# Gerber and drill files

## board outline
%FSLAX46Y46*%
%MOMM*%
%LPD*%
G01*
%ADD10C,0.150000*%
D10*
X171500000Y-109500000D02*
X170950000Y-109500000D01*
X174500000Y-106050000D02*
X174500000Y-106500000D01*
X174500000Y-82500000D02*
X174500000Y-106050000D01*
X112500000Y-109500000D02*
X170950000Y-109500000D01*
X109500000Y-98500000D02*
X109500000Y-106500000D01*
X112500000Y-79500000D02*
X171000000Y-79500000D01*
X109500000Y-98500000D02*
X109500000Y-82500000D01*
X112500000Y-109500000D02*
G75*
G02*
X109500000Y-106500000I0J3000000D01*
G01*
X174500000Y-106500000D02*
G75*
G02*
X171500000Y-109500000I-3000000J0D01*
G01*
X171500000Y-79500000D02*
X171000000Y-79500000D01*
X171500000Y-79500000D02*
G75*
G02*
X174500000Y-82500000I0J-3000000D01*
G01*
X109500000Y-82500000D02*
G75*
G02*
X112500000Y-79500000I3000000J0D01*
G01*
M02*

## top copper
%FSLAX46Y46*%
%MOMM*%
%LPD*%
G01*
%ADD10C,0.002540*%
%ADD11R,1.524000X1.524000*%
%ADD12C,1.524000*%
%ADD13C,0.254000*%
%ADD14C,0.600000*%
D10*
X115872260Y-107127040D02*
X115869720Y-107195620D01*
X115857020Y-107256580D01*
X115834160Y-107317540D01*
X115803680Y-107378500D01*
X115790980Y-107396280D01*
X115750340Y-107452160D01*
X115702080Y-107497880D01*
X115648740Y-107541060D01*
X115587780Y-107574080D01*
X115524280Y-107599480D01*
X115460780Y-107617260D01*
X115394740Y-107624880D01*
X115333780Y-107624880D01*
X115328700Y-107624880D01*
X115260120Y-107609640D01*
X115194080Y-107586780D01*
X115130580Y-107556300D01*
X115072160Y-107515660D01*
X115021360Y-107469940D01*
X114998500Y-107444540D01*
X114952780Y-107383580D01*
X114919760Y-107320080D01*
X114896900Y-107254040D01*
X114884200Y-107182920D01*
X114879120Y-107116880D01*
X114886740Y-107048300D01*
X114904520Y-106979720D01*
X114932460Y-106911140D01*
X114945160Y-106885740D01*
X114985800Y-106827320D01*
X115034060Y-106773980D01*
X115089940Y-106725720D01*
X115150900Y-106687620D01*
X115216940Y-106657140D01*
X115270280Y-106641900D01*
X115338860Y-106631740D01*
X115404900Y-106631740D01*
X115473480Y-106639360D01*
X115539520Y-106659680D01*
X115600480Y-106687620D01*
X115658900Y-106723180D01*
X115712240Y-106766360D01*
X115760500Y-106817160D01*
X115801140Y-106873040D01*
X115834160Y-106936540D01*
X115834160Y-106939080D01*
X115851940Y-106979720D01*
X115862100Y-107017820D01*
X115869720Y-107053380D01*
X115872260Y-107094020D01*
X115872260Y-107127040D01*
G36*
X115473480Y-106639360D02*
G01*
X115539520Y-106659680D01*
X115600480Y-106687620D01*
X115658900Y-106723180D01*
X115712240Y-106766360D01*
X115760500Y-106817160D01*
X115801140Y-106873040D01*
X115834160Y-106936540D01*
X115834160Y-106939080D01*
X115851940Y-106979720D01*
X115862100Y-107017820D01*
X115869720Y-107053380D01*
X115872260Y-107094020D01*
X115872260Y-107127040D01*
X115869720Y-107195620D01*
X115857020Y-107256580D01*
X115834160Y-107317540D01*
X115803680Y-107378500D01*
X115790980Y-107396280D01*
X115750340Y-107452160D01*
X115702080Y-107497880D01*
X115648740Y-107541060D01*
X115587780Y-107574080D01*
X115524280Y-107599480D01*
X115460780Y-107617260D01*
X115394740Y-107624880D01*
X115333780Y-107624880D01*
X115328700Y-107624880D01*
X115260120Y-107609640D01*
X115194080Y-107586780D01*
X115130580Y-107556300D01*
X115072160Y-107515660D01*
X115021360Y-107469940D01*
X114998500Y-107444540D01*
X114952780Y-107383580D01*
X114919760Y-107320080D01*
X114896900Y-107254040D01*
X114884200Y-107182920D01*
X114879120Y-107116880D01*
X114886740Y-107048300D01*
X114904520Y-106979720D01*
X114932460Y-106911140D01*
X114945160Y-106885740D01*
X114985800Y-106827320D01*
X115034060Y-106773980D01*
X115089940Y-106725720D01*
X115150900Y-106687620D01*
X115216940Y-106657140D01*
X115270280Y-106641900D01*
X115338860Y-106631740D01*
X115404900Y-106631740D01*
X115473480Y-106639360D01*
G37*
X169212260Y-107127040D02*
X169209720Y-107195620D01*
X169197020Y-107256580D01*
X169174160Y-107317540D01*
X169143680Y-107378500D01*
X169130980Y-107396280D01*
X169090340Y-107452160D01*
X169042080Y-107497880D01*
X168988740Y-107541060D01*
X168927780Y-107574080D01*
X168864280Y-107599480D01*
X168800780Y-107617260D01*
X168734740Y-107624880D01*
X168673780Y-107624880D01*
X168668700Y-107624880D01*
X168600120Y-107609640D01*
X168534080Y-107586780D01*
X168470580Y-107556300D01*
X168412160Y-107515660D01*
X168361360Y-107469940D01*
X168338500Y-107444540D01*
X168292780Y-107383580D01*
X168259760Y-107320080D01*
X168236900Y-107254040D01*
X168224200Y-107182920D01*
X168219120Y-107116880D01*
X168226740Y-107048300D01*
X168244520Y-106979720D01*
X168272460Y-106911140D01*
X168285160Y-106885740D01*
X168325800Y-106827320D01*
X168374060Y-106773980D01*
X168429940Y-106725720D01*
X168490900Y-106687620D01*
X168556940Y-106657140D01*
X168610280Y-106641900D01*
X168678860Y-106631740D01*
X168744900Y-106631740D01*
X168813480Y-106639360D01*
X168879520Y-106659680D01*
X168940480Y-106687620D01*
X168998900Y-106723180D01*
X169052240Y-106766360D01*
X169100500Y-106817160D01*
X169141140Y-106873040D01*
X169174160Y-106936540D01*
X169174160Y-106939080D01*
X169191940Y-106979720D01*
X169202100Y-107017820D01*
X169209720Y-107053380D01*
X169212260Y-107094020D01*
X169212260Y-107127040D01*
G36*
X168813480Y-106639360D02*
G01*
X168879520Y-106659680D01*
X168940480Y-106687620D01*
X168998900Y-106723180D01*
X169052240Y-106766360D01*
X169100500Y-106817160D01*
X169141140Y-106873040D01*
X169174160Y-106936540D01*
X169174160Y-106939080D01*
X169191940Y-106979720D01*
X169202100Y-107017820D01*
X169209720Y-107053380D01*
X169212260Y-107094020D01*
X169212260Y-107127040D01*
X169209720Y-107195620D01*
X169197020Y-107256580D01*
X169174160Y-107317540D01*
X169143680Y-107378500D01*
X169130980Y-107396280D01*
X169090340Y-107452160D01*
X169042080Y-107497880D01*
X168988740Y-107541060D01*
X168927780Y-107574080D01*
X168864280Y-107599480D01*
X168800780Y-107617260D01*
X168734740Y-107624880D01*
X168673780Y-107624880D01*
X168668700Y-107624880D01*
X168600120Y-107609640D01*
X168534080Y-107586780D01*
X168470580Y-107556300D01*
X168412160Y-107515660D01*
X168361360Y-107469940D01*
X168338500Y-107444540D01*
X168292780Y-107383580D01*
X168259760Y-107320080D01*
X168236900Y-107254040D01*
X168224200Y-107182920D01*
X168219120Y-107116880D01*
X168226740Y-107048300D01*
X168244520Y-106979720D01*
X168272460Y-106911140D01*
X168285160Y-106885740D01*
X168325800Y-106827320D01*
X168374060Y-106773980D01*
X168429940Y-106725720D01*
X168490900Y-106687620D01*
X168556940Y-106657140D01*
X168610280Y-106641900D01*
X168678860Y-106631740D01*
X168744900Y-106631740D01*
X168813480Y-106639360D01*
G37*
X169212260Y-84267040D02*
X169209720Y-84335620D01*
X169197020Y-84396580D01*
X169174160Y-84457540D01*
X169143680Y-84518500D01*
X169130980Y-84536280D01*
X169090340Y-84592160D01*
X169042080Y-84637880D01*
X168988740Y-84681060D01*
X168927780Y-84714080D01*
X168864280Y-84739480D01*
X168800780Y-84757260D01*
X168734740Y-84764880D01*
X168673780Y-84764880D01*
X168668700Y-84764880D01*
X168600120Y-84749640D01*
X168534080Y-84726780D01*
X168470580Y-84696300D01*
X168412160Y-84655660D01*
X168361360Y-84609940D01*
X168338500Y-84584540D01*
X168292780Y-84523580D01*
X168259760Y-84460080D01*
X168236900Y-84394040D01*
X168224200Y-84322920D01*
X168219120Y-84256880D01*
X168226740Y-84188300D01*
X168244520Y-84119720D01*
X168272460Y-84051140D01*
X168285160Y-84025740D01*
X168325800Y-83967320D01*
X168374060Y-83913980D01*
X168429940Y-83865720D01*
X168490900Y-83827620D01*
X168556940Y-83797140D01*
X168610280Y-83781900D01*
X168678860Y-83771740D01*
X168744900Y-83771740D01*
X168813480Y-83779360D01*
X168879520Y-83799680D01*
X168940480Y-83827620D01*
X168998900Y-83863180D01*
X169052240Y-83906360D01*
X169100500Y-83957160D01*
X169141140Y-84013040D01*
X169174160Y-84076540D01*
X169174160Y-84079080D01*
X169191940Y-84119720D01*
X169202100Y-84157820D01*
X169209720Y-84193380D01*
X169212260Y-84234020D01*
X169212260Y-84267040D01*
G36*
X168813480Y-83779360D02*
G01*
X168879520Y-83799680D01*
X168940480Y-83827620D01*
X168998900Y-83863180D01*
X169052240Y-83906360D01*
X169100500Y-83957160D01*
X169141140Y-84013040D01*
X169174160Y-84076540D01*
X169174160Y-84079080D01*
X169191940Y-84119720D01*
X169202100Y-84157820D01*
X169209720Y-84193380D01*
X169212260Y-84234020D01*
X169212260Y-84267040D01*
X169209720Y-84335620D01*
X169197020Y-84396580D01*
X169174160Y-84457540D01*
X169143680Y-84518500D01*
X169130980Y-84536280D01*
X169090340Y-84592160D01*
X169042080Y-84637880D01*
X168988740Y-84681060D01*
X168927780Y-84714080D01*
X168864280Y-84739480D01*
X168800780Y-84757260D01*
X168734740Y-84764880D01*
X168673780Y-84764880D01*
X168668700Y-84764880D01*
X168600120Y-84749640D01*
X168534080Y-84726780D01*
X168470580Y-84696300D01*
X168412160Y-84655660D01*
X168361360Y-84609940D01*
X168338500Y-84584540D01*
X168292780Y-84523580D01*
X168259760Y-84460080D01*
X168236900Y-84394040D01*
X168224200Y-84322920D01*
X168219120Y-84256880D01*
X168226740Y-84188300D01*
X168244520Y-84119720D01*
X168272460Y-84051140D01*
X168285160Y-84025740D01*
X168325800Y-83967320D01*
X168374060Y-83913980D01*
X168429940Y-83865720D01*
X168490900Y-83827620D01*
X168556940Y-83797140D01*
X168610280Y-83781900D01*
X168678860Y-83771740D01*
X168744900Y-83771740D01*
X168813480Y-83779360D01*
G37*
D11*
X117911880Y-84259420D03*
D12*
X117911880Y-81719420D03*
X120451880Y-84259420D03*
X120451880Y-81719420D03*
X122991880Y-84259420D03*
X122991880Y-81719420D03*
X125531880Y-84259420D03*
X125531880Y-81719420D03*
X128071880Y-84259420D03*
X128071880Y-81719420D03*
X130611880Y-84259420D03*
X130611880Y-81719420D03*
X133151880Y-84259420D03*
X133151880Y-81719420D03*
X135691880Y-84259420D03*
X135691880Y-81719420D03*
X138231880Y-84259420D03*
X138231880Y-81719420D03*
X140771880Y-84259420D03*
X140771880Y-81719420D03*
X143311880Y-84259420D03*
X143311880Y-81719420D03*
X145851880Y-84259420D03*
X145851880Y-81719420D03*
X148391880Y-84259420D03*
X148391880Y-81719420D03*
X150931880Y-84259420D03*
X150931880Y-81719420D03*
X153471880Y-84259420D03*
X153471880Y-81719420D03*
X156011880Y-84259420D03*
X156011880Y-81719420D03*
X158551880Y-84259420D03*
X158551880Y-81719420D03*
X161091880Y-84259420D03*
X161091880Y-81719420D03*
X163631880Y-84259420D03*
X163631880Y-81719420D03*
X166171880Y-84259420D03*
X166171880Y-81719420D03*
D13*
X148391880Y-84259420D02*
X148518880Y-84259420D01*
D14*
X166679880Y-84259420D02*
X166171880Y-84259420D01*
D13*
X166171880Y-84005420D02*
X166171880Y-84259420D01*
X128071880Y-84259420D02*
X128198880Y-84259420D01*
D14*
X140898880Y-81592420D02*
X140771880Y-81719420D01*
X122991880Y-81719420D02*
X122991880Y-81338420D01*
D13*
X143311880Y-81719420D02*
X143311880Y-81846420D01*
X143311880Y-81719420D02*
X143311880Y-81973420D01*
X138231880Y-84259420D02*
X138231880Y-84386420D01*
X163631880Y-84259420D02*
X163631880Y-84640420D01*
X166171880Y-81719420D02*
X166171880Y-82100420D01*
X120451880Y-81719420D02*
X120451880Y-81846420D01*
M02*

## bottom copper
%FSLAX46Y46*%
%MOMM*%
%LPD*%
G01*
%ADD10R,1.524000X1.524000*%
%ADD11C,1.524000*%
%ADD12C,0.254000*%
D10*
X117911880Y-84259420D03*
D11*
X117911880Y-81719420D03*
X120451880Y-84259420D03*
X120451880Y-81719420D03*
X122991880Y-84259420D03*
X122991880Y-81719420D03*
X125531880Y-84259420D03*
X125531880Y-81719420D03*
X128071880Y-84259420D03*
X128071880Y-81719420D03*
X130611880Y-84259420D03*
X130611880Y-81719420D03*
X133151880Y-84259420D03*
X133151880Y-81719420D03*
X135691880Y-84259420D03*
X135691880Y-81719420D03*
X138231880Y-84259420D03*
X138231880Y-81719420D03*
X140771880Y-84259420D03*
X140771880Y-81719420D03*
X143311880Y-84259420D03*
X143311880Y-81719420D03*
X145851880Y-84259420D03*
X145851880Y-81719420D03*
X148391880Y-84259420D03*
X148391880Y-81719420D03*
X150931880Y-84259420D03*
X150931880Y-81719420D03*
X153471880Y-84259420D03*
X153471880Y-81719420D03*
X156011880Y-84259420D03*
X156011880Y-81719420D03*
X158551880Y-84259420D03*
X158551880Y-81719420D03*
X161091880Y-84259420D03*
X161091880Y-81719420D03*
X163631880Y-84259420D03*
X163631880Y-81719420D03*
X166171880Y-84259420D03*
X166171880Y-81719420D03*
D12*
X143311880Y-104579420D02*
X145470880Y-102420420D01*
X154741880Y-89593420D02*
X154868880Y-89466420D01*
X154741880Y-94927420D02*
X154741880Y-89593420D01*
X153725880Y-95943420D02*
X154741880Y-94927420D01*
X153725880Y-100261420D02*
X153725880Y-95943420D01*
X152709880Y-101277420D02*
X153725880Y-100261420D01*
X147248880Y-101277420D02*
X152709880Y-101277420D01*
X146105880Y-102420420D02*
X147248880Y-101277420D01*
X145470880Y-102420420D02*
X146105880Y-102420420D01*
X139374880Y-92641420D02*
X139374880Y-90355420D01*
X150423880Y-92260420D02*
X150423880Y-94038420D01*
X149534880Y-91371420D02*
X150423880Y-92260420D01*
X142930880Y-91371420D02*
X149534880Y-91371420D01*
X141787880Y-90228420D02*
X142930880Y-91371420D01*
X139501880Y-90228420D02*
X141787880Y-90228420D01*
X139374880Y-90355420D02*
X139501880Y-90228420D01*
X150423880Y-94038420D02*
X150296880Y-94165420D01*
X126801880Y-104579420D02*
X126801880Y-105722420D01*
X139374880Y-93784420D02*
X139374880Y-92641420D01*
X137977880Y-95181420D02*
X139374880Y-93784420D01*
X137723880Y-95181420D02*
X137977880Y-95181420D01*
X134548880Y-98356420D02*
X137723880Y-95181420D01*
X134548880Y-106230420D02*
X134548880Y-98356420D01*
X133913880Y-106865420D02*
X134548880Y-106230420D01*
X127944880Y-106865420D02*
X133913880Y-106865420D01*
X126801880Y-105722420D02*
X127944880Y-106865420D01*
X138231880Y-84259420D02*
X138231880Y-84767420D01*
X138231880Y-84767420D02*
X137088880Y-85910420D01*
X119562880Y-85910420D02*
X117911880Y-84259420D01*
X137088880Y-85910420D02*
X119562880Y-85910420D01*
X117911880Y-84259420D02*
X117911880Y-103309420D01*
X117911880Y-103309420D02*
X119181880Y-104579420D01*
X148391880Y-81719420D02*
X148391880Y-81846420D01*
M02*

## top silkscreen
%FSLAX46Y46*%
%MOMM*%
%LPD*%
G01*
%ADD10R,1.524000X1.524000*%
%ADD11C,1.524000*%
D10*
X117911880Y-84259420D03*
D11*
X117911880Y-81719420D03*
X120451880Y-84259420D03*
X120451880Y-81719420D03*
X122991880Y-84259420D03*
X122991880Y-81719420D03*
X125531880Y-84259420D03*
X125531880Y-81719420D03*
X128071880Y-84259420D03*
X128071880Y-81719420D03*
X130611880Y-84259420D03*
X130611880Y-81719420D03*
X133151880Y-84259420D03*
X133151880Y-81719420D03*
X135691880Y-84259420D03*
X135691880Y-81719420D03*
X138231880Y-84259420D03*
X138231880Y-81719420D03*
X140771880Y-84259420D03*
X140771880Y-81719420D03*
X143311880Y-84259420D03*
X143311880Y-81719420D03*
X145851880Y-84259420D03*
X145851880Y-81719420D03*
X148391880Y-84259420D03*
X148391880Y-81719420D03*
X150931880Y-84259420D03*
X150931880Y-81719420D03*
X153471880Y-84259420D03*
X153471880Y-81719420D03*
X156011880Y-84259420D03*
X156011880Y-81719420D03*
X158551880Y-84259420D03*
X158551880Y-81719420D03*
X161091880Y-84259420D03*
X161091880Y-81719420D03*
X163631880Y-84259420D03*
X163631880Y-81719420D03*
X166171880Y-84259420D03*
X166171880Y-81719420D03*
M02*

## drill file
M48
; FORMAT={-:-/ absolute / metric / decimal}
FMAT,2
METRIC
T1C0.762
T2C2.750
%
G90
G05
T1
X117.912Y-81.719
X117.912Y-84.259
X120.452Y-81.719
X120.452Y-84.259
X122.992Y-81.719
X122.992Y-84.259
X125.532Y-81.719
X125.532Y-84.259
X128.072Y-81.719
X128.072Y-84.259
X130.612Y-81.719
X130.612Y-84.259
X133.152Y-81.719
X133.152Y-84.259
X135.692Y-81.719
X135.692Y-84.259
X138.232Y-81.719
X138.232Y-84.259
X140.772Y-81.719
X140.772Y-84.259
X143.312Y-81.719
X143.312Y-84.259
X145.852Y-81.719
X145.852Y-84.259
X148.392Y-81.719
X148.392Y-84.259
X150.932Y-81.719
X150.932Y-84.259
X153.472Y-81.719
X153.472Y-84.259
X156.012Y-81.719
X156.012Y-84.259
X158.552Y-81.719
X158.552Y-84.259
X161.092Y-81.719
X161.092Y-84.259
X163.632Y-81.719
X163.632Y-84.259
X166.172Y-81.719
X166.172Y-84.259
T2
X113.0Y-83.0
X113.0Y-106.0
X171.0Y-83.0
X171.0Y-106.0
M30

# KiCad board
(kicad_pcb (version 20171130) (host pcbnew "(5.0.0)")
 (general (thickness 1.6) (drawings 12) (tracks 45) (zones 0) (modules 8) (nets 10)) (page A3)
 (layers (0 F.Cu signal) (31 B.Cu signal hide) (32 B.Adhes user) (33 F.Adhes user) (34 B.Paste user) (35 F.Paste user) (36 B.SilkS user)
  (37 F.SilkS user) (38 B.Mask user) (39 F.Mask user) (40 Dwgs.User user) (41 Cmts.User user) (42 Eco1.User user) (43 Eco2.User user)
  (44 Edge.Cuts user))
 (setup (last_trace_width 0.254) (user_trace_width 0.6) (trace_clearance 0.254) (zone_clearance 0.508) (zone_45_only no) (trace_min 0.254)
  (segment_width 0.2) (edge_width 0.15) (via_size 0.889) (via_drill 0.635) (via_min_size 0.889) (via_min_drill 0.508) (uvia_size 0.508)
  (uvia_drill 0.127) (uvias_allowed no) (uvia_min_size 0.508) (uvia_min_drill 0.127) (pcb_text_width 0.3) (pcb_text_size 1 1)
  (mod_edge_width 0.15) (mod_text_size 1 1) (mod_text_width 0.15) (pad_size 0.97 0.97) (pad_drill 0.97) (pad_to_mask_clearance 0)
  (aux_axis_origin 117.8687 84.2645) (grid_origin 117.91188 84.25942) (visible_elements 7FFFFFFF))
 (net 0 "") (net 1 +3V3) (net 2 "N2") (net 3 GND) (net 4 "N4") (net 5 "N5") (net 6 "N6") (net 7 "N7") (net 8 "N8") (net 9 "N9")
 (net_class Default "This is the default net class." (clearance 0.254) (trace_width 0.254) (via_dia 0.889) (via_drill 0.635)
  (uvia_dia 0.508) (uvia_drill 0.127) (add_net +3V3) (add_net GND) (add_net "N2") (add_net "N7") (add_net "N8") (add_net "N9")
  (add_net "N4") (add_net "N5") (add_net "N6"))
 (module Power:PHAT (layer F.Cu) (at 117.91188 82.98942 90)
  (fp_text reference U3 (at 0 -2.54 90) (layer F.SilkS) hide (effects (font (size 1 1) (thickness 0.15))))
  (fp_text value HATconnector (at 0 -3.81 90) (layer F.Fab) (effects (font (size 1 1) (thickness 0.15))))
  (pad 1 thru_hole rect (at -1.27 0 90) (size 1.524 1.524) (drill 0.762) (layers *.Cu *.Mask F.SilkS) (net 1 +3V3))
  (pad 2 thru_hole circle (at 1.27 0 90) (size 1.524 1.524) (drill 0.762) (layers *.Cu *.Mask F.SilkS) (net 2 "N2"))
  (pad 3 thru_hole circle (at -1.27 2.54 90) (size 1.524 1.524) (drill 0.762) (layers *.Cu *.Mask F.SilkS))
  (pad 4 thru_hole circle (at 1.27 2.54 90) (size 1.524 1.524) (drill 0.762) (layers *.Cu *.Mask F.SilkS) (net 2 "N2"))
  (pad 5 thru_hole circle (at -1.27 5.08 90) (size 1.524 1.524) (drill 0.762) (layers *.Cu *.Mask F.SilkS))
  (pad 6 thru_hole circle (at 1.27 5.08 90) (size 1.524 1.524) (drill 0.762) (layers *.Cu *.Mask F.SilkS) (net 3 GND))
  (pad 7 thru_hole circle (at -1.27 7.62 90) (size 1.524 1.524) (drill 0.762) (layers *.Cu *.Mask F.SilkS))
  (pad 8 thru_hole circle (at 1.27 7.62 90) (size 1.524 1.524) (drill 0.762) (layers *.Cu *.Mask F.SilkS))
  (pad 9 thru_hole circle (at -1.27 10.16 90) (size 1.524 1.524) (drill 0.762) (layers *.Cu *.Mask F.SilkS) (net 3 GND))
  (pad 10 thru_hole circle (at 1.27 10.16 90) (size 1.524 1.524) (drill 0.762) (layers *.Cu *.Mask F.SilkS))
  (pad 11 thru_hole circle (at -1.27 12.7 90) (size 1.524 1.524) (drill 0.762) (layers *.Cu *.Mask F.SilkS))
  (pad 12 thru_hole circle (at 1.27 12.7 90) (size 1.524 1.524) (drill 0.762) (layers *.Cu *.Mask F.SilkS))
  (pad 13 thru_hole circle (at -1.27 15.24 90) (size 1.524 1.524) (drill 0.762) (layers *.Cu *.Mask F.SilkS))
  (pad 14 thru_hole circle (at 1.27 15.24 90) (size 1.524 1.524) (drill 0.762) (layers *.Cu *.Mask F.SilkS) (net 3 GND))
  (pad 15 thru_hole circle (at -1.27 17.78 90) (size 1.524 1.524) (drill 0.762) (layers *.Cu *.Mask F.SilkS))
  (pad 16 thru_hole circle (at 1.27 17.78 90) (size 1.524 1.524) (drill 0.762) (layers *.Cu *.Mask F.SilkS))
  (pad 17 thru_hole circle (at -1.27 20.32 90) (size 1.524 1.524) (drill 0.762) (layers *.Cu *.Mask F.SilkS) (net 1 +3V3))
  (pad 18 thru_hole circle (at 1.27 20.32 90) (size 1.524 1.524) (drill 0.762) (layers *.Cu *.Mask F.SilkS))
  (pad 19 thru_hole circle (at -1.27 22.86 90) (size 1.524 1.524) (drill 0.762) (layers *.Cu *.Mask F.SilkS))
  (pad 20 thru_hole circle (at 1.27 22.86 90) (size 1.524 1.524) (drill 0.762) (layers *.Cu *.Mask F.SilkS) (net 3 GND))
  (pad 21 thru_hole circle (at -1.27 25.4 90) (size 1.524 1.524) (drill 0.762) (layers *.Cu *.Mask F.SilkS))
  (pad 22 thru_hole circle (at 1.27 25.4 90) (size 1.524 1.524) (drill 0.762) (layers *.Cu *.Mask F.SilkS) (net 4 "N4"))
  (pad 23 thru_hole circle (at -1.27 27.94 90) (size 1.524 1.524) (drill 0.762) (layers *.Cu *.Mask F.SilkS))
  (pad 24 thru_hole circle (at 1.27 27.94 90) (size 1.524 1.524) (drill 0.762) (layers *.Cu *.Mask F.SilkS))
  (pad 25 thru_hole circle (at -1.27 30.48 90) (size 1.524 1.524) (drill 0.762) (layers *.Cu *.Mask F.SilkS) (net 3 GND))
  (pad 26 thru_hole circle (at 1.27 30.48 90) (size 1.524 1.524) (drill 0.762) (layers *.Cu *.Mask F.SilkS) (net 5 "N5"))
  (pad 27 thru_hole circle (at -1.27 33.02 90) (size 1.524 1.524) (drill 0.762) (layers *.Cu *.Mask F.SilkS))
  (pad 28 thru_hole circle (at 1.27 33.02 90) (size 1.524 1.524) (drill 0.762) (layers *.Cu *.Mask F.SilkS))
  (pad 29 thru_hole circle (at -1.27 35.56 90) (size 1.524 1.524) (drill 0.762) (layers *.Cu *.Mask F.SilkS))
  (pad 30 thru_hole circle (at 1.27 35.56 90) (size 1.524 1.524) (drill 0.762) (layers *.Cu *.Mask F.SilkS) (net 3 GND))
  (pad 31 thru_hole circle (at -1.27 38.1 90) (size 1.524 1.524) (drill 0.762) (layers *.Cu *.Mask F.SilkS))
  (pad 32 thru_hole circle (at 1.27 38.1 90) (size 1.524 1.524) (drill 0.762) (layers *.Cu *.Mask F.SilkS))
  (pad 33 thru_hole circle (at -1.27 40.64 90) (size 1.524 1.524) (drill 0.762) (layers *.Cu *.Mask F.SilkS))
  (pad 34 thru_hole circle (at 1.27 40.64 90) (size 1.524 1.524) (drill 0.762) (layers *.Cu *.Mask F.SilkS) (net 3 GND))
  (pad 35 thru_hole circle (at -1.27 43.18 90) (size 1.524 1.524) (drill 0.762) (layers *.Cu *.Mask F.SilkS) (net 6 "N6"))
  (pad 36 thru_hole circle (at 1.27 43.18 90) (size 1.524 1.524) (drill 0.762) (layers *.Cu *.Mask F.SilkS))
  (pad 37 thru_hole circle (at -1.27 45.72 90) (size 1.524 1.524) (drill 0.762) (layers *.Cu *.Mask F.SilkS) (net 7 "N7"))
  (pad 38 thru_hole circle (at 1.27 45.72 90) (size 1.524 1.524) (drill 0.762) (layers *.Cu *.Mask F.SilkS) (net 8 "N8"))
  (pad 39 thru_hole circle (at -1.27 48.26 90) (size 1.524 1.524) (drill 0.762) (layers *.Cu *.Mask F.SilkS) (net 3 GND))
  (pad 40 thru_hole circle (at 1.27 48.26 90) (size 1.524 1.524) (drill 0.762) (layers *.Cu *.Mask F.SilkS) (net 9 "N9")))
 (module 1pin (layer F.Cu) (at 171 106)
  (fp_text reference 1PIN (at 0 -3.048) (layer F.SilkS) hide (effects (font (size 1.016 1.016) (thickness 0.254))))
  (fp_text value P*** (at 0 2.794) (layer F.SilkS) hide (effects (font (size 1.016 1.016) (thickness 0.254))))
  (pad "" np_thru_hole circle (at 0 0) (size 2.75 2.75) (drill 2.75) (layers *.Cu)))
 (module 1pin (layer F.Cu) (at 113 106)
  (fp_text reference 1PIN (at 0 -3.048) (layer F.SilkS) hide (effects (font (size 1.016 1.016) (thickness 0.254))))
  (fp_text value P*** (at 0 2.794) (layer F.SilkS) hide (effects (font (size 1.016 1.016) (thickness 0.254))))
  (pad "" np_thru_hole circle (at 0 0) (size 2.75 2.75) (drill 2.75) (layers *.Cu)))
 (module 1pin (layer F.Cu) (at 171 83)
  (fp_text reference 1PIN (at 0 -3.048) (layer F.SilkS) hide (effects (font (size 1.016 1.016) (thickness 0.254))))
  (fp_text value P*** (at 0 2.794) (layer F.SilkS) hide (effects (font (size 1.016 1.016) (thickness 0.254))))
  (pad "" np_thru_hole circle (at 0 0) (size 2.75 2.75) (drill 2.75) (layers *.Cu)))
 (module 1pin (layer F.Cu) (at 113 83)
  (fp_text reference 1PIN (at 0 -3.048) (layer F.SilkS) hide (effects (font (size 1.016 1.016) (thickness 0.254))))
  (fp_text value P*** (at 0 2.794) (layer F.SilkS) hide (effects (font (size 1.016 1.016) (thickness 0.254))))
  (pad "" np_thru_hole circle (at 0 0) (size 2.75 2.75) (drill 2.75) (layers *.Cu)))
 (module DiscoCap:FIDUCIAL (layer F.Cu) (at 115.37188 107.11942)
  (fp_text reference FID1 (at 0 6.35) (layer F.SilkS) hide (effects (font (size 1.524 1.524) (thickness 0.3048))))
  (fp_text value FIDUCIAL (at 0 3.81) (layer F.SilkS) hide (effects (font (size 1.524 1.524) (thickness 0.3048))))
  (fp_poly
   (pts (xy 0.50038 0.00762) (xy 0.49784 0.0762) (xy 0.48514 0.13716) (xy 0.46228 0.19812) (xy 0.4318 0.25908) (xy 0.4191 0.27686)
    (xy 0.37846 0.33274) (xy 0.3302 0.37846) (xy 0.27686 0.42164) (xy 0.2159 0.45466) (xy 0.1524 0.48006) (xy 0.0889 0.49784)
    (xy 0.02286 0.50546) (xy -0.0381 0.50546) (xy -0.04318 0.50546) (xy -0.11176 0.49022) (xy -0.1778 0.46736) (xy -0.2413 0.43688)
    (xy -0.29972 0.39624) (xy -0.35052 0.35052) (xy -0.37338 0.32512) (xy -0.4191 0.26416) (xy -0.45212 0.20066) (xy -0.47498 0.13462)
    (xy -0.48768 0.0635) (xy -0.49276 -0.00254) (xy -0.48514 -0.07112) (xy -0.46736 -0.1397) (xy -0.43942 -0.20828) (xy -0.42672 -0.23368)
    (xy -0.38608 -0.2921) (xy -0.33782 -0.34544) (xy -0.28194 -0.3937) (xy -0.22098 -0.4318) (xy -0.15494 -0.46228) (xy -0.1016 -0.47752)
    (xy -0.03302 -0.48768) (xy 0.03302 -0.48768) (xy 0.1016 -0.48006) (xy 0.16764 -0.45974) (xy 0.2286 -0.4318) (xy 0.28702 -0.39624)
    (xy 0.34036 -0.35306) (xy 0.38862 -0.30226) (xy 0.42926 -0.24638) (xy 0.46228 -0.18288) (xy 0.46228 -0.18034) (xy 0.48006 -0.1397)
    (xy 0.49022 -0.1016) (xy 0.49784 -0.06604) (xy 0.50038 -0.0254) (xy 0.50038 0.00762))
   (layer F.Cu) (width 0.00254)))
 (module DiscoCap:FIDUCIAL (layer F.Cu) (at 168.71188 107.11942)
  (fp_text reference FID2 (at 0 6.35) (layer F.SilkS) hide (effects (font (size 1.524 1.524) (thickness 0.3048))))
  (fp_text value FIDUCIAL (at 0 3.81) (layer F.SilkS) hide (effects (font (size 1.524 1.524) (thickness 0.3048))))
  (fp_poly
   (pts (xy 0.50038 0.00762) (xy 0.49784 0.0762) (xy 0.48514 0.13716) (xy 0.46228 0.19812) (xy 0.4318 0.25908) (xy 0.4191 0.27686)
    (xy 0.37846 0.33274) (xy 0.3302 0.37846) (xy 0.27686 0.42164) (xy 0.2159 0.45466) (xy 0.1524 0.48006) (xy 0.0889 0.49784)
    (xy 0.02286 0.50546) (xy -0.0381 0.50546) (xy -0.04318 0.50546) (xy -0.11176 0.49022) (xy -0.1778 0.46736) (xy -0.2413 0.43688)
    (xy -0.29972 0.39624) (xy -0.35052 0.35052) (xy -0.37338 0.32512) (xy -0.4191 0.26416) (xy -0.45212 0.20066) (xy -0.47498 0.13462)
    (xy -0.48768 0.0635) (xy -0.49276 -0.00254) (xy -0.48514 -0.07112) (xy -0.46736 -0.1397) (xy -0.43942 -0.20828) (xy -0.42672 -0.23368)
    (xy -0.38608 -0.2921) (xy -0.33782 -0.34544) (xy -0.28194 -0.3937) (xy -0.22098 -0.4318) (xy -0.15494 -0.46228) (xy -0.1016 -0.47752)
    (xy -0.03302 -0.48768) (xy 0.03302 -0.48768) (xy 0.1016 -0.48006) (xy 0.16764 -0.45974) (xy 0.2286 -0.4318) (xy 0.28702 -0.39624)
    (xy 0.34036 -0.35306) (xy 0.38862 -0.30226) (xy 0.42926 -0.24638) (xy 0.46228 -0.18288) (xy 0.46228 -0.18034) (xy 0.48006 -0.1397)
    (xy 0.49022 -0.1016) (xy 0.49784 -0.06604) (xy 0.50038 -0.0254) (xy 0.50038 0.00762))
   (layer F.Cu) (width 0.00254)))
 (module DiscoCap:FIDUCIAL (layer F.Cu) (at 168.71188 84.25942)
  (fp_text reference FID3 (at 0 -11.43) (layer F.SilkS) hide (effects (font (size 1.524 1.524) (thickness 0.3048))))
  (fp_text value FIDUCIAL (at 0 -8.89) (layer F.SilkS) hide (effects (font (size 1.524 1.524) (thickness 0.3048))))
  (fp_poly
   (pts (xy 0.50038 0.00762) (xy 0.49784 0.0762) (xy 0.48514 0.13716) (xy 0.46228 0.19812) (xy 0.4318 0.25908) (xy 0.4191 0.27686)
    (xy 0.37846 0.33274) (xy 0.3302 0.37846) (xy 0.27686 0.42164) (xy 0.2159 0.45466) (xy 0.1524 0.48006) (xy 0.0889 0.49784)
    (xy 0.02286 0.50546) (xy -0.0381 0.50546) (xy -0.04318 0.50546) (xy -0.11176 0.49022) (xy -0.1778 0.46736) (xy -0.2413 0.43688)
    (xy -0.29972 0.39624) (xy -0.35052 0.35052) (xy -0.37338 0.32512) (xy -0.4191 0.26416) (xy -0.45212 0.20066) (xy -0.47498 0.13462)
    (xy -0.48768 0.0635) (xy -0.49276 -0.00254) (xy -0.48514 -0.07112) (xy -0.46736 -0.1397) (xy -0.43942 -0.20828) (xy -0.42672 -0.23368)
    (xy -0.38608 -0.2921) (xy -0.33782 -0.34544) (xy -0.28194 -0.3937) (xy -0.22098 -0.4318) (xy -0.15494 -0.46228) (xy -0.1016 -0.47752)
    (xy -0.03302 -0.48768) (xy 0.03302 -0.48768) (xy 0.1016 -0.48006) (xy 0.16764 -0.45974) (xy 0.2286 -0.4318) (xy 0.28702 -0.39624)
    (xy 0.34036 -0.35306) (xy 0.38862 -0.30226) (xy 0.42926 -0.24638) (xy 0.46228 -0.18288) (xy 0.46228 -0.18034) (xy 0.48006 -0.1397)
    (xy 0.49022 -0.1016) (xy 0.49784 -0.06604) (xy 0.50038 -0.0254) (xy 0.50038 0.00762))
   (layer F.Cu) (width 0.00254)))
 (gr_line (start 171.5 109.5) (end 170.95 109.5) (angle 90) (layer Edge.Cuts) (width 0.15))
 (gr_line (start 174.5 106.05) (end 174.5 106.5) (angle 90) (layer Edge.Cuts) (width 0.15))
 (gr_line (start 174.5 82.5) (end 174.5 106.05) (angle 90) (layer Edge.Cuts) (width 0.15))
 (gr_line (start 112.5 109.5) (end 170.95 109.5) (angle 90) (layer Edge.Cuts) (width 0.15))
 (gr_line (start 109.5 98.5) (end 109.5 106.5) (angle 90) (layer Edge.Cuts) (width 0.15))
 (gr_line (start 112.5 79.5) (end 171 79.5) (angle 90) (layer Edge.Cuts) (width 0.15))
 (gr_line (start 109.5 98.5) (end 109.5 82.5) (angle 90) (layer Edge.Cuts) (width 0.15))
 (gr_arc (start 112.5 106.5) (end 112.5 109.5) (angle 90) (layer Edge.Cuts) (width 0.15))
 (gr_arc (start 171.5 106.5) (end 174.5 106.5) (angle 90) (layer Edge.Cuts) (width 0.15))
 (gr_line (start 171.5 79.5) (end 171 79.5) (angle 90) (layer Edge.Cuts) (width 0.15))
 (gr_arc (start 171.5 82.5) (end 171.5 79.5) (angle 90) (layer Edge.Cuts) (width 0.15))
 (gr_arc (start 112.5 82.5) (end 109.5 82.5) (angle 90) (layer Edge.Cuts) (width 0.15))
 (segment (start 143.31188 104.57942) (end 145.47088 102.42042) (width 0.254) (layer B.Cu) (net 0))
 (segment (start 154.74188 89.59342) (end 154.86888 89.46642) (width 0.254) (layer B.Cu) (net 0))
 (segment (start 154.74188 94.92742) (end 154.74188 89.59342) (width 0.254) (layer B.Cu) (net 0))
 (segment (start 153.72588 95.94342) (end 154.74188 94.92742) (width 0.254) (layer B.Cu) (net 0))
 (segment (start 153.72588 100.26142) (end 153.72588 95.94342) (width 0.254) (layer B.Cu) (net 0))
 (segment (start 152.70988 101.27742) (end 153.72588 100.26142) (width 0.254) (layer B.Cu) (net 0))
 (segment (start 147.24888 101.27742) (end 152.70988 101.27742) (width 0.254) (layer B.Cu) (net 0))
 (segment (start 146.10588 102.42042) (end 147.24888 101.27742) (width 0.254) (layer B.Cu) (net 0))
 (segment (start 145.47088 102.42042) (end 146.10588 102.42042) (width 0.254) (layer B.Cu) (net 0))
 (segment (start 139.37488 92.64142) (end 139.37488 90.35542) (width 0.254) (layer B.Cu) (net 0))
 (segment (start 150.42388 92.26042) (end 150.42388 94.03842) (width 0.254) (layer B.Cu) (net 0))
 (segment (start 149.53488 91.37142) (end 150.42388 92.26042) (width 0.254) (layer B.Cu) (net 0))
 (segment (start 142.93088 91.37142) (end 149.53488 91.37142) (width 0.254) (layer B.Cu) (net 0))
 (segment (start 141.78788 90.22842) (end 142.93088 91.37142) (width 0.254) (layer B.Cu) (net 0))
 (segment (start 139.50188 90.22842) (end 141.78788 90.22842) (width 0.254) (layer B.Cu) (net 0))
 (segment (start 139.37488 90.35542) (end 139.50188 90.22842) (width 0.254) (layer B.Cu) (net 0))
 (segment (start 150.42388 94.03842) (end 150.29688 94.16542) (width 0.254) (layer B.Cu) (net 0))
 (segment (start 126.80188 104.57942) (end 126.80188 105.72242) (width 0.254) (layer B.Cu) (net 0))
 (segment (start 139.37488 93.78442) (end 139.37488 92.64142) (width 0.254) (layer B.Cu) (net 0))
 (segment (start 137.97788 95.18142) (end 139.37488 93.78442) (width 0.254) (layer B.Cu) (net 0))
 (segment (start 137.72388 95.18142) (end 137.97788 95.18142) (width 0.254) (layer B.Cu) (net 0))
 (segment (start 134.54888 98.35642) (end 137.72388 95.18142) (width 0.254) (layer B.Cu) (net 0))
 (segment (start 134.54888 106.23042) (end 134.54888 98.35642) (width 0.254) (layer B.Cu) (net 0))
 (segment (start 133.91388 106.86542) (end 134.54888 106.23042) (width 0.254) (layer B.Cu) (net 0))
 (segment (start 127.94488 106.86542) (end 133.91388 106.86542) (width 0.254) (layer B.Cu) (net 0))
 (segment (start 126.80188 105.72242) (end 127.94488 106.86542) (width 0.254) (layer B.Cu) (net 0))
 (segment (start 148.39188 84.25942) (end 148.51888 84.25942) (width 0.254) (layer F.Cu) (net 3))
 (segment (start 166.67988 84.25942) (end 166.17188 84.25942) (width 0.6) (layer F.Cu) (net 3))
 (segment (start 166.17188 84.00542) (end 166.17188 84.25942) (width 0.254) (layer F.Cu) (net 3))
 (segment (start 128.07188 84.25942) (end 128.19888 84.25942) (width 0.254) (layer F.Cu) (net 3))
 (segment (start 140.89888 81.59242) (end 140.77188 81.71942) (width 0.6) (layer F.Cu) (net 3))
 (segment (start 122.99188 81.71942) (end 122.99188 81.33842) (width 0.6) (layer F.Cu) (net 3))
 (segment (start 143.31188 81.71942) (end 143.31188 81.84642) (width 0.254) (layer F.Cu) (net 4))
 (segment (start 143.31188 81.71942) (end 143.31188 81.97342) (width 0.254) (layer F.Cu) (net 4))
 (segment (start 138.23188 84.25942) (end 138.23188 84.76742) (width 0.254) (layer B.Cu) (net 1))
 (segment (start 138.23188 84.76742) (end 137.08888 85.91042) (width 0.254) (layer B.Cu) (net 1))
 (segment (start 119.56288 85.91042) (end 117.91188 84.25942) (width 0.254) (layer B.Cu) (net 1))
 (segment (start 137.08888 85.91042) (end 119.56288 85.91042) (width 0.254) (layer B.Cu) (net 1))
 (segment (start 117.91188 84.25942) (end 117.91188 103.30942) (width 0.254) (layer B.Cu) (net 1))
 (segment (start 117.91188 103.30942) (end 119.18188 104.57942) (width 0.254) (layer B.Cu) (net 1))
 (segment (start 138.23188 84.25942) (end 138.23188 84.38642) (width 0.254) (layer F.Cu) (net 1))
 (segment (start 163.63188 84.25942) (end 163.63188 84.64042) (width 0.254) (layer F.Cu) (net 7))
 (segment (start 166.17188 81.71942) (end 166.17188 82.10042) (width 0.254) (layer F.Cu) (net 9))
 (segment (start 148.39188 81.71942) (end 148.39188 81.84642) (width 0.254) (layer B.Cu) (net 5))
 (segment (start 120.45188 81.71942) (end 120.45188 81.84642) (width 0.254) (layer F.Cu) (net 2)))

